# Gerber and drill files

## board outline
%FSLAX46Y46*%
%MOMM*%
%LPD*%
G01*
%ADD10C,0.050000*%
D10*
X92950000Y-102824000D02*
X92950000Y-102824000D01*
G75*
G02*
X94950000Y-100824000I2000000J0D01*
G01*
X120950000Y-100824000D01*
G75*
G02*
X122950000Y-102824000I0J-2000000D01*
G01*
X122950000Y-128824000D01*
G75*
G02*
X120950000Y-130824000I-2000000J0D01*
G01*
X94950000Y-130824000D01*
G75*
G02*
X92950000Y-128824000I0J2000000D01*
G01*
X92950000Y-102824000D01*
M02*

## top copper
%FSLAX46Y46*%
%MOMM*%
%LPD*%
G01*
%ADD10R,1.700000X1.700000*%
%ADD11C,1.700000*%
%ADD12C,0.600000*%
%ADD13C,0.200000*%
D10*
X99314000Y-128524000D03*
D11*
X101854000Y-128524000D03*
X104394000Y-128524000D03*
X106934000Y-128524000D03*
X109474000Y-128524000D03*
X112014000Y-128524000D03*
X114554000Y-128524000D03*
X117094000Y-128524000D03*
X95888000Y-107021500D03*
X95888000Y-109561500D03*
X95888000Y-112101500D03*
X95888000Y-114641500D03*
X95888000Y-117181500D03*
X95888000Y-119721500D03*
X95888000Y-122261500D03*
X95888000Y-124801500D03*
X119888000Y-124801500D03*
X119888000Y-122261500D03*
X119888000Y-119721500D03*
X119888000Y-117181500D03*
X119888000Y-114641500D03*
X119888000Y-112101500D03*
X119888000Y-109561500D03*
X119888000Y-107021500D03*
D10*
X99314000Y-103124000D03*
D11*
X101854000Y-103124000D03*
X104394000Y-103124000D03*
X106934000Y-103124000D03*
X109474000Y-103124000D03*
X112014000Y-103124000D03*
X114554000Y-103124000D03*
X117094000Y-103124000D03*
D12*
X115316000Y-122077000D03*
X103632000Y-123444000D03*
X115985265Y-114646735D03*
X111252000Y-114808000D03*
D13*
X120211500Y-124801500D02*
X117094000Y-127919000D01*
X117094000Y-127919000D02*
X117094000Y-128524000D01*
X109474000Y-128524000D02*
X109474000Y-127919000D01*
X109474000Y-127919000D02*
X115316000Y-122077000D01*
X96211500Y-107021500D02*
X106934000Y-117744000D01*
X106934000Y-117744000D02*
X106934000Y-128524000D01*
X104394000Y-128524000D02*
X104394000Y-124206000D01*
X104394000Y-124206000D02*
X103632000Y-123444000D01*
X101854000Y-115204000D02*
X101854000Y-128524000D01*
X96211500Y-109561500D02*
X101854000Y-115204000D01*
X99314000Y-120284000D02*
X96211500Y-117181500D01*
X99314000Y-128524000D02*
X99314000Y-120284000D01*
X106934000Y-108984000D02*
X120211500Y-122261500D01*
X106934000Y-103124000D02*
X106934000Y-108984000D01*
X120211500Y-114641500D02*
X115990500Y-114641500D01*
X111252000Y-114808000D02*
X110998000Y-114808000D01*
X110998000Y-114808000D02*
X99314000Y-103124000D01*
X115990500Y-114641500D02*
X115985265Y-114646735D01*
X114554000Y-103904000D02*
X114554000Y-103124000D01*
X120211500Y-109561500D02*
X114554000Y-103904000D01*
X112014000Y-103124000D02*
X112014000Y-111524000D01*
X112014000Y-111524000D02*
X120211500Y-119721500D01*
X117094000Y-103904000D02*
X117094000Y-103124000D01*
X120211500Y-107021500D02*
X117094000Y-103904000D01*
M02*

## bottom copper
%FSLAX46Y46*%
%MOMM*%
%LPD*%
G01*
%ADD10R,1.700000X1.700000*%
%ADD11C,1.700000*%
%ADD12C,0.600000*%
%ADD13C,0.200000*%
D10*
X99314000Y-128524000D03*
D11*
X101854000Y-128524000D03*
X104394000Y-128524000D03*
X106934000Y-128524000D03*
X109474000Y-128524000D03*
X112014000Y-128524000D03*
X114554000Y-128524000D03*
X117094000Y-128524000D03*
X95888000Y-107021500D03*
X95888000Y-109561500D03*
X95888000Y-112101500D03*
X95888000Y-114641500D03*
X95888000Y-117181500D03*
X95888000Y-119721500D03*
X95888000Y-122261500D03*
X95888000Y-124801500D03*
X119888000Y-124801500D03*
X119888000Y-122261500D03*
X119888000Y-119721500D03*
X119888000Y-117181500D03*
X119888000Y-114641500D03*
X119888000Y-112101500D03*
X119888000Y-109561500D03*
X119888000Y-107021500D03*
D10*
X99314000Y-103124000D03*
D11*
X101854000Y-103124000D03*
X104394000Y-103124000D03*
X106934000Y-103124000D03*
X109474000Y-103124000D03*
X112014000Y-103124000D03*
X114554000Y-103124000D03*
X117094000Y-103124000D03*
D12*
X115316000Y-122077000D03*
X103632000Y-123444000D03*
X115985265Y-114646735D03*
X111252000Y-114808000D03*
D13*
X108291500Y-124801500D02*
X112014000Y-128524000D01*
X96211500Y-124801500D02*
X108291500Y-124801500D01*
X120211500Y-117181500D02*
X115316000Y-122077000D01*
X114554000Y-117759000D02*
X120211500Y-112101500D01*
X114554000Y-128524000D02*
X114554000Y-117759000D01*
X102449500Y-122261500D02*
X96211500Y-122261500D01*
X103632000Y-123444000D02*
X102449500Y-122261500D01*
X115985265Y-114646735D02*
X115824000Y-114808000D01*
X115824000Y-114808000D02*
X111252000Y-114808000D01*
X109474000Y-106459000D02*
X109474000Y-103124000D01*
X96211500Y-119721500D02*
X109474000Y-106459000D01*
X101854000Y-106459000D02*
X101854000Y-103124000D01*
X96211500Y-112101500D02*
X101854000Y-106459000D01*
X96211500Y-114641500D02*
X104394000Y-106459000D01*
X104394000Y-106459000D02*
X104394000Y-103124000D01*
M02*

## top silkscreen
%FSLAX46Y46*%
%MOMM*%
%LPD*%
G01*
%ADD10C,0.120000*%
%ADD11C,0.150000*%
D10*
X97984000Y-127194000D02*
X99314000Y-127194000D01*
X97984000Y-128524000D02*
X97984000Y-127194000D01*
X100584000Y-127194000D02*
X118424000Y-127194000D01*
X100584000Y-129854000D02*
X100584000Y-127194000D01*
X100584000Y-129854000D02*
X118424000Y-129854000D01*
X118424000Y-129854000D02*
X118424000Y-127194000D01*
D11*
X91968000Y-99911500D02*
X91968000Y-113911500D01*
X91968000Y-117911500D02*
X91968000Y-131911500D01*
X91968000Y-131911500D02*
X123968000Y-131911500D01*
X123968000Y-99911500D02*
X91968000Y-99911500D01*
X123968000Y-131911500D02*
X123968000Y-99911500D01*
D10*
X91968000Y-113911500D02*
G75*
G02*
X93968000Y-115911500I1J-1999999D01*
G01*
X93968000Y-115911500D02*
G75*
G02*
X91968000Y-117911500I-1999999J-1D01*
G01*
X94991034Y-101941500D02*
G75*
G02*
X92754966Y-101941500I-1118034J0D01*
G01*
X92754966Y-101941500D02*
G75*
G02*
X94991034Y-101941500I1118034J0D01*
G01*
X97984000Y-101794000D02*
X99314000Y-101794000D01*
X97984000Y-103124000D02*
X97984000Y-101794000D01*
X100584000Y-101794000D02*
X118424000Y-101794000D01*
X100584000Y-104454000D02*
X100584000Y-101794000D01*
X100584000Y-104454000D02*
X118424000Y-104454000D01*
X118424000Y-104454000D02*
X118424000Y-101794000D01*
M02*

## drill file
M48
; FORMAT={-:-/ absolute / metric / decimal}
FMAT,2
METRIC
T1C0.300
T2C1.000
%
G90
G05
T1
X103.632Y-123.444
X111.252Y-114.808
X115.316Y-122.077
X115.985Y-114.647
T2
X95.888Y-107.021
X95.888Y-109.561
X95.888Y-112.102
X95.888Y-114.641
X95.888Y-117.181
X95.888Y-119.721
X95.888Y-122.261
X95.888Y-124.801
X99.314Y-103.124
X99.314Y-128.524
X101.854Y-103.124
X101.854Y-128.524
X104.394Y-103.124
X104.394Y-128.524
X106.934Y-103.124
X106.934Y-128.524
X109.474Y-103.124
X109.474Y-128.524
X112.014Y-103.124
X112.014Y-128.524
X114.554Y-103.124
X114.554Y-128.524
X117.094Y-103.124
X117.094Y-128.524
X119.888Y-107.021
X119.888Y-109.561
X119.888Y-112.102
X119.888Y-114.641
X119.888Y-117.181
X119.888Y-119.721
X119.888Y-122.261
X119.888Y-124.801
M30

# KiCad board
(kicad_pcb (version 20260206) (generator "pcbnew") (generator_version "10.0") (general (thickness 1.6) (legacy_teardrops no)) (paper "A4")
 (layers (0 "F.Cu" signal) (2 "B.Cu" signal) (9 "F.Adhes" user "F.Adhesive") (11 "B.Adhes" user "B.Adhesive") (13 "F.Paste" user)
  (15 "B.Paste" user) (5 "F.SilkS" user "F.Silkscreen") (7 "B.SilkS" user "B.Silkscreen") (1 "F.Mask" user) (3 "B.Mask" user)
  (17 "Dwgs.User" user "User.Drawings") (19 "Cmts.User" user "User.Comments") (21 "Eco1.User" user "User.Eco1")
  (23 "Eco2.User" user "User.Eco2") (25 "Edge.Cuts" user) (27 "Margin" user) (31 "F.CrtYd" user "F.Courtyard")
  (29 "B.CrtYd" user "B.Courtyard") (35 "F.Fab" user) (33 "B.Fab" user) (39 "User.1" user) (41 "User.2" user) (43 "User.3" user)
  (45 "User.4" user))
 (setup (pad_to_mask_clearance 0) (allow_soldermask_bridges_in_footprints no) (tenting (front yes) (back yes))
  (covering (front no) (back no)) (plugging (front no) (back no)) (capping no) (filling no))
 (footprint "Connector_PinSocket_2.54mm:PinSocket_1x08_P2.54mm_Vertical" (layer "F.Cu") (at 99.314 128.524 90)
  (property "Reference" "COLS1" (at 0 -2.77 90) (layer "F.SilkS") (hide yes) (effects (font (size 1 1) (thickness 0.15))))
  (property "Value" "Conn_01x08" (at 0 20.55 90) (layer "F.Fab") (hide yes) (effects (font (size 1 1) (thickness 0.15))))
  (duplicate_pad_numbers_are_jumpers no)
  (fp_line (start 1.33 -1.33) (end 1.33 0) (stroke (width 0.12) (type solid)) (layer "F.SilkS"))
  (fp_line (start 0 -1.33) (end 1.33 -1.33) (stroke (width 0.12) (type solid)) (layer "F.SilkS"))
  (fp_line (start 1.33 1.27) (end 1.33 19.11) (stroke (width 0.12) (type solid)) (layer "F.SilkS"))
  (fp_line (start -1.33 1.27) (end 1.33 1.27) (stroke (width 0.12) (type solid)) (layer "F.SilkS"))
  (fp_line (start -1.33 1.27) (end -1.33 19.11) (stroke (width 0.12) (type solid)) (layer "F.SilkS"))
  (fp_line (start -1.33 19.11) (end 1.33 19.11) (stroke (width 0.12) (type solid)) (layer "F.SilkS"))
  (pad "1" thru_hole rect (at 0 0 90) (size 1.7 1.7) (drill 1) (layers "*.Cu" "*.Mask") (remove_unused_layers no) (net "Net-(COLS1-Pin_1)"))
  (pad "2" thru_hole circle (at 0 2.54 90) (size 1.7 1.7) (drill 1) (layers "*.Cu" "*.Mask") (remove_unused_layers no)
   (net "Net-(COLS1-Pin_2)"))
  (pad "3" thru_hole circle (at 0 5.08 90) (size 1.7 1.7) (drill 1) (layers "*.Cu" "*.Mask") (remove_unused_layers no)
   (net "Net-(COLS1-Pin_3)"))
  (pad "4" thru_hole circle (at 0 7.62 90) (size 1.7 1.7) (drill 1) (layers "*.Cu" "*.Mask") (remove_unused_layers no)
   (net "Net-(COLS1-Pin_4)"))
  (pad "5" thru_hole circle (at 0 10.16 90) (size 1.7 1.7) (drill 1) (layers "*.Cu" "*.Mask") (remove_unused_layers no)
   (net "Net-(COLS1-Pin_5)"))
  (pad "6" thru_hole circle (at 0 12.7 90) (size 1.7 1.7) (drill 1) (layers "*.Cu" "*.Mask") (remove_unused_layers no)
   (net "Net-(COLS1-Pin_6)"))
  (pad "7" thru_hole circle (at 0 15.24 90) (size 1.7 1.7) (drill 1) (layers "*.Cu" "*.Mask") (remove_unused_layers no)
   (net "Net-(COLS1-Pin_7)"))
  (pad "8" thru_hole circle (at 0 17.78 90) (size 1.7 1.7) (drill 1) (layers "*.Cu" "*.Mask") (remove_unused_layers no)
   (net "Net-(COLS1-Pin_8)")))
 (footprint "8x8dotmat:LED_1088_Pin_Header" (layer "F.Cu") (at 91.968 99.9115)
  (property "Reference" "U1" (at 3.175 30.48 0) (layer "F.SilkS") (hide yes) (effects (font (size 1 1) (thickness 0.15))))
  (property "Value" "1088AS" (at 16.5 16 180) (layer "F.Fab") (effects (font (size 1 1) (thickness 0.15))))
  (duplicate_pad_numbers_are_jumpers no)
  (fp_line (start 0 0) (end 0 14) (stroke (width 0.15) (type solid)) (layer "F.SilkS"))
  (fp_line (start 0 18) (end 0 32) (stroke (width 0.15) (type solid)) (layer "F.SilkS"))
  (fp_line (start 0 32) (end 32 32) (stroke (width 0.15) (type solid)) (layer "F.SilkS"))
  (fp_line (start 32 0) (end 0 0) (stroke (width 0.15) (type solid)) (layer "F.SilkS"))
  (fp_line (start 32 32) (end 32 0) (stroke (width 0.15) (type solid)) (layer "F.SilkS"))
  (fp_arc (start 0 14) (mid 1.414214 14.585786) (end 2 16) (stroke (width 0.12) (type solid)) (layer "F.SilkS"))
  (fp_arc (start 2 16) (mid 1.414214 17.414214) (end 0 18) (stroke (width 0.12) (type solid)) (layer "F.SilkS"))
  (fp_circle (center 1.905 2.03) (end 1.905 0.911966) (stroke (width 0.12) (type solid)) (fill no) (layer "F.SilkS"))
  (pad "1" thru_hole circle (at 3.92 7.11 270) (size 1.7 1.7) (drill 1) (layers "*.Cu" "*.Mask") (remove_unused_layers no)
   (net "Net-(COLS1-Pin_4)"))
  (pad "2" thru_hole circle (at 3.92 9.65 270) (size 1.7 1.7) (drill 1) (layers "*.Cu" "*.Mask") (remove_unused_layers no)
   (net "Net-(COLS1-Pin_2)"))
  (pad "3" thru_hole circle (at 3.92 12.19 270) (size 1.7 1.7) (drill 1) (layers "*.Cu" "*.Mask") (remove_unused_layers no)
   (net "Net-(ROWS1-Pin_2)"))
  (pad "4" thru_hole circle (at 3.92 14.73 270) (size 1.7 1.7) (drill 1) (layers "*.Cu" "*.Mask") (remove_unused_layers no)
   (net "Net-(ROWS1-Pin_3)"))
  (pad "5" thru_hole circle (at 3.92 17.27 270) (size 1.7 1.7) (drill 1) (layers "*.Cu" "*.Mask") (remove_unused_layers no)
   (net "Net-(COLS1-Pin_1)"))
  (pad "6" thru_hole circle (at 3.92 19.81 270) (size 1.7 1.7) (drill 1) (layers "*.Cu" "*.Mask") (remove_unused_layers no)
   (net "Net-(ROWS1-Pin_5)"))
  (pad "7" thru_hole circle (at 3.92 22.35 270) (size 1.7 1.7) (drill 1) (layers "*.Cu" "*.Mask") (remove_unused_layers no)
   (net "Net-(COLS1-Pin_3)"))
  (pad "8" thru_hole circle (at 3.92 24.89 270) (size 1.7 1.7) (drill 1) (layers "*.Cu" "*.Mask") (remove_unused_layers no)
   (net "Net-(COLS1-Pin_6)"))
  (pad "9" thru_hole circle (at 27.92 24.89 270) (size 1.7 1.7) (drill 1) (layers "*.Cu" "*.Mask") (remove_unused_layers no)
   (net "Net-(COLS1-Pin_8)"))
  (pad "10" thru_hole circle (at 27.92 22.35 270) (size 1.7 1.7) (drill 1) (layers "*.Cu" "*.Mask") (remove_unused_layers no)
   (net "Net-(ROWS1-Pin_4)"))
  (pad "11" thru_hole circle (at 27.92 19.81 270) (size 1.7 1.7) (drill 1) (layers "*.Cu" "*.Mask") (remove_unused_layers no)
   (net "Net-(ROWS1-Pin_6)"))
  (pad "12" thru_hole circle (at 27.92 17.27 270) (size 1.7 1.7) (drill 1) (layers "*.Cu" "*.Mask") (remove_unused_layers no)
   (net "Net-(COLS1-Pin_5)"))
  (pad "13" thru_hole circle (at 27.92 14.73 270) (size 1.7 1.7) (drill 1) (layers "*.Cu" "*.Mask") (remove_unused_layers no)
   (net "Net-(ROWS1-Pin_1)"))
  (pad "14" thru_hole circle (at 27.92 12.19 270) (size 1.7 1.7) (drill 1) (layers "*.Cu" "*.Mask") (remove_unused_layers no)
   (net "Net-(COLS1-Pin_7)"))
  (pad "15" thru_hole circle (at 27.92 9.65 270) (size 1.7 1.7) (drill 1) (layers "*.Cu" "*.Mask") (remove_unused_layers no)
   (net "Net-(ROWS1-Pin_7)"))
  (pad "16" thru_hole circle (at 27.92 7.11 270) (size 1.7 1.7) (drill 1) (layers "*.Cu" "*.Mask") (remove_unused_layers no)
   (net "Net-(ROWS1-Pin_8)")))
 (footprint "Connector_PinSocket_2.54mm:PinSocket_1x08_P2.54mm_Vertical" (layer "F.Cu") (at 99.314 103.124 90)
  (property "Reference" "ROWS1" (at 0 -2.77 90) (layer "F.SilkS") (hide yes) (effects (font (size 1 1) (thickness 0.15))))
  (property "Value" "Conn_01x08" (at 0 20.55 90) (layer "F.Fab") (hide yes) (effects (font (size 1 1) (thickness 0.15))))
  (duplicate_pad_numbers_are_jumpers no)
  (fp_line (start 1.33 -1.33) (end 1.33 0) (stroke (width 0.12) (type solid)) (layer "F.SilkS"))
  (fp_line (start 0 -1.33) (end 1.33 -1.33) (stroke (width 0.12) (type solid)) (layer "F.SilkS"))
  (fp_line (start 1.33 1.27) (end 1.33 19.11) (stroke (width 0.12) (type solid)) (layer "F.SilkS"))
  (fp_line (start -1.33 1.27) (end 1.33 1.27) (stroke (width 0.12) (type solid)) (layer "F.SilkS"))
  (fp_line (start -1.33 1.27) (end -1.33 19.11) (stroke (width 0.12) (type solid)) (layer "F.SilkS"))
  (fp_line (start -1.33 19.11) (end 1.33 19.11) (stroke (width 0.12) (type solid)) (layer "F.SilkS"))
  (pad "1" thru_hole rect (at 0 0 90) (size 1.7 1.7) (drill 1) (layers "*.Cu" "*.Mask") (remove_unused_layers no) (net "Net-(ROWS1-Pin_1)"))
  (pad "2" thru_hole circle (at 0 2.54 90) (size 1.7 1.7) (drill 1) (layers "*.Cu" "*.Mask") (remove_unused_layers no)
   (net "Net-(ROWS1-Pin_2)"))
  (pad "3" thru_hole circle (at 0 5.08 90) (size 1.7 1.7) (drill 1) (layers "*.Cu" "*.Mask") (remove_unused_layers no)
   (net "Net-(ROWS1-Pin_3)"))
  (pad "4" thru_hole circle (at 0 7.62 90) (size 1.7 1.7) (drill 1) (layers "*.Cu" "*.Mask") (remove_unused_layers no)
   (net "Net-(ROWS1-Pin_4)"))
  (pad "5" thru_hole circle (at 0 10.16 90) (size 1.7 1.7) (drill 1) (layers "*.Cu" "*.Mask") (remove_unused_layers no)
   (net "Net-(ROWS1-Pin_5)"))
  (pad "6" thru_hole circle (at 0 12.7 90) (size 1.7 1.7) (drill 1) (layers "*.Cu" "*.Mask") (remove_unused_layers no)
   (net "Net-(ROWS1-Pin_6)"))
  (pad "7" thru_hole circle (at 0 15.24 90) (size 1.7 1.7) (drill 1) (layers "*.Cu" "*.Mask") (remove_unused_layers no)
   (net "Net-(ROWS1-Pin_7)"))
  (pad "8" thru_hole circle (at 0 17.78 90) (size 1.7 1.7) (drill 1) (layers "*.Cu" "*.Mask") (remove_unused_layers no)
   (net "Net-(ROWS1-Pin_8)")))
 (gr_rect (start 92.95 100.824) (end 122.95 130.824) (radius 2) (stroke (width 0.05) (type solid)) (fill no) (layer "Edge.Cuts"))
 (segment (start 108.2915 124.8015) (end 112.014 128.524) (width 0.2) (layer "B.Cu") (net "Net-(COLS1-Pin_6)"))
 (segment (start 96.2115 124.8015) (end 108.2915 124.8015) (width 0.2) (layer "B.Cu") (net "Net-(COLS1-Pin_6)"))
 (segment (start 120.2115 124.8015) (end 117.094 127.919) (width 0.2) (layer "F.Cu") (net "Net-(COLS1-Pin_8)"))
 (segment (start 117.094 127.919) (end 117.094 128.524) (width 0.2) (layer "F.Cu") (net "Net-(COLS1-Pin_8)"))
 (segment (start 109.474 128.524) (end 109.474 127.919) (width 0.2) (layer "F.Cu") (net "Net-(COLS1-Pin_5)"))
 (segment (start 109.474 127.919) (end 115.316 122.077) (width 0.2) (layer "F.Cu") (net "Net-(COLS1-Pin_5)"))
 (via (at 115.316 122.077) (size 0.6) (drill 0.3) (layers "F.Cu" "B.Cu") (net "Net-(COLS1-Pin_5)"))
 (segment (start 120.2115 117.1815) (end 115.316 122.077) (width 0.2) (layer "B.Cu") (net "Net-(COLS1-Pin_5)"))
 (segment (start 114.554 117.759) (end 120.2115 112.1015) (width 0.2) (layer "B.Cu") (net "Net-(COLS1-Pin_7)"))
 (segment (start 114.554 128.524) (end 114.554 117.759) (width 0.2) (layer "B.Cu") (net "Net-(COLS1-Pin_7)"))
 (segment (start 96.2115 107.0215) (end 106.934 117.744) (width 0.2) (layer "F.Cu") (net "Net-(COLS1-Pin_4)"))
 (segment (start 106.934 117.744) (end 106.934 128.524) (width 0.2) (layer "F.Cu") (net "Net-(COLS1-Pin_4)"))
 (segment (start 104.394 128.524) (end 104.394 124.206) (width 0.2) (layer "F.Cu") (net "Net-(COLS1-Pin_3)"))
 (segment (start 104.394 124.206) (end 103.632 123.444) (width 0.2) (layer "F.Cu") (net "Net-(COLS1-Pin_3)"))
 (via (at 103.632 123.444) (size 0.6) (drill 0.3) (layers "F.Cu" "B.Cu") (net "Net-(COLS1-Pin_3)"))
 (segment (start 102.4495 122.2615) (end 96.2115 122.2615) (width 0.2) (layer "B.Cu") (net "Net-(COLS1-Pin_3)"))
 (segment (start 103.632 123.444) (end 102.4495 122.2615) (width 0.2) (layer "B.Cu") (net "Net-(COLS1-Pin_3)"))
 (segment (start 101.854 115.204) (end 101.854 128.524) (width 0.2) (layer "F.Cu") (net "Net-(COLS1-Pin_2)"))
 (segment (start 96.2115 109.5615) (end 101.854 115.204) (width 0.2) (layer "F.Cu") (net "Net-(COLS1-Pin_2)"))
 (segment (start 99.314 120.284) (end 96.2115 117.1815) (width 0.2) (layer "F.Cu") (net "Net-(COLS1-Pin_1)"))
 (segment (start 99.314 128.524) (end 99.314 120.284) (width 0.2) (layer "F.Cu") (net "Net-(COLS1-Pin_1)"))
 (segment (start 106.934 108.984) (end 120.2115 122.2615) (width 0.2) (layer "F.Cu") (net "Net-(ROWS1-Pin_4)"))
 (segment (start 106.934 103.124) (end 106.934 108.984) (width 0.2) (layer "F.Cu") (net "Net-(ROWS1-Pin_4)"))
 (segment (start 120.2115 114.6415) (end 115.9905 114.6415) (width 0.2) (layer "F.Cu") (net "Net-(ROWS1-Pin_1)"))
 (segment (start 111.252 114.808) (end 110.998 114.808) (width 0.2) (layer "F.Cu") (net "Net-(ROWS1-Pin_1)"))
 (segment (start 110.998 114.808) (end 99.314 103.124) (width 0.2) (layer "F.Cu") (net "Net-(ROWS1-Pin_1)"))
 (segment (start 115.9905 114.6415) (end 115.985265 114.646735) (width 0.2) (layer "F.Cu") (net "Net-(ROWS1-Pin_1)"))
 (via (at 115.985265 114.646735) (size 0.6) (drill 0.3) (layers "F.Cu" "B.Cu") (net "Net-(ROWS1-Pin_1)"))
 (via (at 111.252 114.808) (size 0.6) (drill 0.3) (layers "F.Cu" "B.Cu") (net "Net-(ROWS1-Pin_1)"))
 (segment (start 115.985265 114.646735) (end 115.824 114.808) (width 0.2) (layer "B.Cu") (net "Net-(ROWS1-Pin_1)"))
 (segment (start 115.824 114.808) (end 111.252 114.808) (width 0.2) (layer "B.Cu") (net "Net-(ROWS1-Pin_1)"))
 (segment (start 114.554 103.904) (end 114.554 103.124) (width 0.2) (layer "F.Cu") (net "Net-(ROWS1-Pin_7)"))
 (segment (start 120.2115 109.5615) (end 114.554 103.904) (width 0.2) (layer "F.Cu") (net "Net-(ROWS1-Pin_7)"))
 (segment (start 109.474 106.459) (end 109.474 103.124) (width 0.2) (layer "B.Cu") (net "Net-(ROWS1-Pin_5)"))
 (segment (start 96.2115 119.7215) (end 109.474 106.459) (width 0.2) (layer "B.Cu") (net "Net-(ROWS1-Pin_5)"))
 (segment (start 101.854 106.459) (end 101.854 103.124) (width 0.2) (layer "B.Cu") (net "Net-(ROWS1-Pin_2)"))
 (segment (start 96.2115 112.1015) (end 101.854 106.459) (width 0.2) (layer "B.Cu") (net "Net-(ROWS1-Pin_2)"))
 (segment (start 112.014 103.124) (end 112.014 111.524) (width 0.2) (layer "F.Cu") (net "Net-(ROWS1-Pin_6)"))
 (segment (start 112.014 111.524) (end 120.2115 119.7215) (width 0.2) (layer "F.Cu") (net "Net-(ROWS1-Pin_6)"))
 (segment (start 96.2115 114.6415) (end 104.394 106.459) (width 0.2) (layer "B.Cu") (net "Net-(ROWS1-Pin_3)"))
 (segment (start 104.394 106.459) (end 104.394 103.124) (width 0.2) (layer "B.Cu") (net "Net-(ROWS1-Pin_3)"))
 (segment (start 117.094 103.904) (end 117.094 103.124) (width 0.2) (layer "F.Cu") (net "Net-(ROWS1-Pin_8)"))
 (segment (start 120.2115 107.0215) (end 117.094 103.904) (width 0.2) (layer "F.Cu") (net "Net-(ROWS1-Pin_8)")))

